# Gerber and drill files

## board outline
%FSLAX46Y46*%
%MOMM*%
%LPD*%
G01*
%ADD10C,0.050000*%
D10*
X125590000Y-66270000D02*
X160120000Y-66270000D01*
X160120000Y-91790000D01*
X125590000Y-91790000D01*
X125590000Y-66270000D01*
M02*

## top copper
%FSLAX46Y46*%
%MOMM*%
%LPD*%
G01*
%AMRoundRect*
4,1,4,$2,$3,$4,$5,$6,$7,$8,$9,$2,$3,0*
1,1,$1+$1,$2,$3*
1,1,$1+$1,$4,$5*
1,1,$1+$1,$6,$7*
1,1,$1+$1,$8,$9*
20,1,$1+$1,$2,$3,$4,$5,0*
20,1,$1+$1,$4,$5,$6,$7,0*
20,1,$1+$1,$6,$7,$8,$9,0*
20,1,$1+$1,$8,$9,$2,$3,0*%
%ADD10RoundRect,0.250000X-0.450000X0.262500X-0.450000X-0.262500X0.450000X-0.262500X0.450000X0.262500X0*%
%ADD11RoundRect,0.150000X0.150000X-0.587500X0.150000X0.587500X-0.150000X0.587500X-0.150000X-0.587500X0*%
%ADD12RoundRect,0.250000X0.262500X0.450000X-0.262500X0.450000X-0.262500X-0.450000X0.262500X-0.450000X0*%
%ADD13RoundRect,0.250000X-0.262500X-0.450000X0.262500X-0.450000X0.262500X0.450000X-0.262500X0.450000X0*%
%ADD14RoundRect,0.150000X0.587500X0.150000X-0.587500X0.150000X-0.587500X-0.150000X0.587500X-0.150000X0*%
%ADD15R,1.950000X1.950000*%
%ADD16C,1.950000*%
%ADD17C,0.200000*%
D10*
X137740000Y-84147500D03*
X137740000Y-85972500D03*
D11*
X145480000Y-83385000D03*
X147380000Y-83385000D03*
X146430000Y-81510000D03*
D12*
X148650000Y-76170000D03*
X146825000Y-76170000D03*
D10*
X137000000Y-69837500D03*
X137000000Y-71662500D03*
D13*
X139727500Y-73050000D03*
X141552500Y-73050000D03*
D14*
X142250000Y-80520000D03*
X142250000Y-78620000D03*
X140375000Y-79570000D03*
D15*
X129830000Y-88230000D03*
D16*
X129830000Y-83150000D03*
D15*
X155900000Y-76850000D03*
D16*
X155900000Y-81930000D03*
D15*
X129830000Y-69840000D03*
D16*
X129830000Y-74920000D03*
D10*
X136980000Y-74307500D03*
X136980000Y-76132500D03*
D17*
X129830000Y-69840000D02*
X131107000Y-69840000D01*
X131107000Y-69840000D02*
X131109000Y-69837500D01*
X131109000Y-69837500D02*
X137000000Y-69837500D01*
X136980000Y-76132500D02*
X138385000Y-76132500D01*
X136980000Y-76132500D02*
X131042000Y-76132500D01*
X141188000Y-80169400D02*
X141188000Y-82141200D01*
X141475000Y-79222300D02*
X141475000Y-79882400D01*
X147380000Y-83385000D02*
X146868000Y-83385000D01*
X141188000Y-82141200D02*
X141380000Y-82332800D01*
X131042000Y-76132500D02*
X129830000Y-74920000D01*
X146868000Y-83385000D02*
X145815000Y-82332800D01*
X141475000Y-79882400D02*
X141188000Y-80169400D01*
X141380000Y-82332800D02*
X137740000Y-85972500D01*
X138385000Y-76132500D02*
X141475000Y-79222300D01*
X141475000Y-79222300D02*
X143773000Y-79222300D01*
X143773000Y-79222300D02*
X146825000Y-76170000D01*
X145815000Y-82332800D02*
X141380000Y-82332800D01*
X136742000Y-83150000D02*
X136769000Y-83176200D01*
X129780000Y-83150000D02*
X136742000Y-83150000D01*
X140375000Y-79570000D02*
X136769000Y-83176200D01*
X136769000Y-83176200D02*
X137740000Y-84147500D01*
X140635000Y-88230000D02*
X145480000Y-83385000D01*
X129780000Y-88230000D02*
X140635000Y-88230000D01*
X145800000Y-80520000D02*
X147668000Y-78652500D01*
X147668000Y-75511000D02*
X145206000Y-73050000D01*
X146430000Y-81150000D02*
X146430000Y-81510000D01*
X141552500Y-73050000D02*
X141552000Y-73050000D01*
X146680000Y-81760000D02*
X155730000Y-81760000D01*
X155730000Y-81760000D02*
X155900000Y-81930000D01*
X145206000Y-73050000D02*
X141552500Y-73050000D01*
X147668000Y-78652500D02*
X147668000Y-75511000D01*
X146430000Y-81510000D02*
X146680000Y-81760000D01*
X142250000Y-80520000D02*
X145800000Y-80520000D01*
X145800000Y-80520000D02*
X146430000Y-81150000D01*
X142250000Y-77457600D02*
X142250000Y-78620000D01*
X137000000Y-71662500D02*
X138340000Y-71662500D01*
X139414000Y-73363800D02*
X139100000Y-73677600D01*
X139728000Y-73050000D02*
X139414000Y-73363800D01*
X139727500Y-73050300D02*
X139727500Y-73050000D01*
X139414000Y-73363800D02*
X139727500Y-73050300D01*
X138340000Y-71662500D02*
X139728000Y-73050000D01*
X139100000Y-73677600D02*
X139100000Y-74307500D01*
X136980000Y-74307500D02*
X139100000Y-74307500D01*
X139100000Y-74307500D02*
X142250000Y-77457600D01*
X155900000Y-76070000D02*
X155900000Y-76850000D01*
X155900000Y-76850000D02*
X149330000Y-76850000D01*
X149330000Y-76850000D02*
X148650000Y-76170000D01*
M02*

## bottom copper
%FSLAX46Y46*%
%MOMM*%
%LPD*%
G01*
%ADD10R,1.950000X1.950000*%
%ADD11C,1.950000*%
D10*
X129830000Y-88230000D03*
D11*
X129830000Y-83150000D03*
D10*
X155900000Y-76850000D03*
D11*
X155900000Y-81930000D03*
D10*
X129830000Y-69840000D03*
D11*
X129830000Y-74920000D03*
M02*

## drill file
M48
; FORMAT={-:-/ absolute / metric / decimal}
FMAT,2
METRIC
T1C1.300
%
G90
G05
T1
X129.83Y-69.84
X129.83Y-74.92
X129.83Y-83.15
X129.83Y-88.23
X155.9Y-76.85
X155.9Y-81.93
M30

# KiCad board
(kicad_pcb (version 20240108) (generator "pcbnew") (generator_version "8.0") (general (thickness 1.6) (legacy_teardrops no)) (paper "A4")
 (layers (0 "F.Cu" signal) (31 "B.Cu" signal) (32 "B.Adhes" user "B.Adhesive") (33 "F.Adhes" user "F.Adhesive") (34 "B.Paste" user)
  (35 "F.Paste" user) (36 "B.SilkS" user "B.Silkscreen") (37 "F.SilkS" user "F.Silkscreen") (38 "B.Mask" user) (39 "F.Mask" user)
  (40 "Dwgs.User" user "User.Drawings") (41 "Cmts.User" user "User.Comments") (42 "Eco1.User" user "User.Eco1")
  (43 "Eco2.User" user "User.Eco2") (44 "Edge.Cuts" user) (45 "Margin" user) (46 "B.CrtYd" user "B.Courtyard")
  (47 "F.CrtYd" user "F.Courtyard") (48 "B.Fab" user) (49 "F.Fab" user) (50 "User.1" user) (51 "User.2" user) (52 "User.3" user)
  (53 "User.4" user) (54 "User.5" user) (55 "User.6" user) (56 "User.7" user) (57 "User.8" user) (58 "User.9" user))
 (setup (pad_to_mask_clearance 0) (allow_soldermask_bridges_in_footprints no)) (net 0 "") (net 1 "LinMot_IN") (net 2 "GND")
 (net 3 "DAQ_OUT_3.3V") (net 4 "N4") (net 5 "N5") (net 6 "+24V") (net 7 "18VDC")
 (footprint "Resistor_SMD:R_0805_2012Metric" (layer "F.Cu") (at 137.74 85.06 -90)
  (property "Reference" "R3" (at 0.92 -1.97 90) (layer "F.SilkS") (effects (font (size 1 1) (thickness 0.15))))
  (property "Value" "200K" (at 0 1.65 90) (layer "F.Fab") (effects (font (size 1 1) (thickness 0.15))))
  (pad "1" smd roundrect (at -0.9125 0 270) (size 1.025 1.4) (layers "F.Cu" "F.Paste" "F.Mask") (roundrect_rratio 0.243902)
   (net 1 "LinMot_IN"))
  (pad "2" smd roundrect (at 0.9125 0 270) (size 1.025 1.4) (layers "F.Cu" "F.Paste" "F.Mask") (roundrect_rratio 0.243902) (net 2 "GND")))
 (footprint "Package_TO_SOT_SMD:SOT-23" (layer "F.Cu") (at 146.43 82.4475 90)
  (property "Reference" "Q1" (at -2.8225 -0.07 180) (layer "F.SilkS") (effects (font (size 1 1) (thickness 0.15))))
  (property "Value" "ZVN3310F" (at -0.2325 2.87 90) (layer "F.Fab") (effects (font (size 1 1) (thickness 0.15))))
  (pad "1" smd roundrect (at -0.9375 -0.95 90) (size 1.475 0.6) (layers "F.Cu" "F.Paste" "F.Mask") (roundrect_rratio 0.25)
   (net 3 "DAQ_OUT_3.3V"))
  (pad "2" smd roundrect (at -0.9375 0.95 90) (size 1.475 0.6) (layers "F.Cu" "F.Paste" "F.Mask") (roundrect_rratio 0.25) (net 2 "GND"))
  (pad "3" smd roundrect (at 0.9375 0 90) (size 1.475 0.6) (layers "F.Cu" "F.Paste" "F.Mask") (roundrect_rratio 0.25) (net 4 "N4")))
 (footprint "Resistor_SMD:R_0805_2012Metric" (layer "F.Cu") (at 147.7375 76.17 180)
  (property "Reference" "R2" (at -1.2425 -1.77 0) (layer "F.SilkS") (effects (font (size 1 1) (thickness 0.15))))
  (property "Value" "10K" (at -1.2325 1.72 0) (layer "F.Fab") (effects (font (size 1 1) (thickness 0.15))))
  (pad "1" smd roundrect (at -0.9125 0 180) (size 1.025 1.4) (layers "F.Cu" "F.Paste" "F.Mask") (roundrect_rratio 0.243902) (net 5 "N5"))
  (pad "2" smd roundrect (at 0.9125 0 180) (size 1.025 1.4) (layers "F.Cu" "F.Paste" "F.Mask") (roundrect_rratio 0.243902) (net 2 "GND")))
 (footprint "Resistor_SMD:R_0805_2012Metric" (layer "F.Cu") (at 137 70.75 -90)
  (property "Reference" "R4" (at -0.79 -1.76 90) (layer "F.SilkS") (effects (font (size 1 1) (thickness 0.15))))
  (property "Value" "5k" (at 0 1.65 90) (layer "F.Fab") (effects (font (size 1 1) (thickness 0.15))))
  (pad "1" smd roundrect (at -0.9125 0 270) (size 1.025 1.4) (layers "F.Cu" "F.Paste" "F.Mask") (roundrect_rratio 0.243902) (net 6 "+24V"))
  (pad "2" smd roundrect (at 0.9125 0 270) (size 1.025 1.4) (layers "F.Cu" "F.Paste" "F.Mask") (roundrect_rratio 0.243902) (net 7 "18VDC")))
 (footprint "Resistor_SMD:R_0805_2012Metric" (layer "F.Cu") (at 140.64 73.05)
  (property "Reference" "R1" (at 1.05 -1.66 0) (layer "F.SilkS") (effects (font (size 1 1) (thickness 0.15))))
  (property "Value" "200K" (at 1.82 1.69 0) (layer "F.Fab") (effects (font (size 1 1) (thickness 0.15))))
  (pad "1" smd roundrect (at -0.9125 0) (size 1.025 1.4) (layers "F.Cu" "F.Paste" "F.Mask") (roundrect_rratio 0.243902) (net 7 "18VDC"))
  (pad "2" smd roundrect (at 0.9125 0) (size 1.025 1.4) (layers "F.Cu" "F.Paste" "F.Mask") (roundrect_rratio 0.243902) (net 4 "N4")))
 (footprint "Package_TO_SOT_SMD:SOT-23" (layer "F.Cu") (at 141.3125 79.57 180)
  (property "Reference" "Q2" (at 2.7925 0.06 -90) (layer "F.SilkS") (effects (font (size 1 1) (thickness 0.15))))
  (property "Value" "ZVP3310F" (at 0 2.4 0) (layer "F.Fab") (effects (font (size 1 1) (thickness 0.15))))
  (pad "1" smd roundrect (at -0.9375 -0.95 180) (size 1.475 0.6) (layers "F.Cu" "F.Paste" "F.Mask") (roundrect_rratio 0.25) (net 4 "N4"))
  (pad "2" smd roundrect (at -0.9375 0.95 180) (size 1.475 0.6) (layers "F.Cu" "F.Paste" "F.Mask") (roundrect_rratio 0.25) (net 7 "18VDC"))
  (pad "3" smd roundrect (at 0.9375 0 180) (size 1.475 0.6) (layers "F.Cu" "F.Paste" "F.Mask") (roundrect_rratio 0.25) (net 1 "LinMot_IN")))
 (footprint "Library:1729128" (layer "F.Cu") (at 129.83 88.23 90)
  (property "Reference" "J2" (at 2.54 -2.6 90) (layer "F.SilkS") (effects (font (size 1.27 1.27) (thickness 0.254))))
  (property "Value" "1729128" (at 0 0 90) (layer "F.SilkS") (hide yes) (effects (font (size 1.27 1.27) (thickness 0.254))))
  (pad "1" thru_hole rect (at 0 0 90) (size 1.95 1.95) (drill 1.3) (layers "*.Cu" "*.Mask") (remove_unused_layers no) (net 3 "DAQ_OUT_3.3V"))
  (pad "2" thru_hole circle (at 5.08 0 90) (size 1.95 1.95) (drill 1.3) (layers "*.Cu" "*.Mask") (remove_unused_layers no)
   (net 1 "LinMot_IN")))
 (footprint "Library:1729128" (layer "F.Cu") (at 155.9 76.85 -90)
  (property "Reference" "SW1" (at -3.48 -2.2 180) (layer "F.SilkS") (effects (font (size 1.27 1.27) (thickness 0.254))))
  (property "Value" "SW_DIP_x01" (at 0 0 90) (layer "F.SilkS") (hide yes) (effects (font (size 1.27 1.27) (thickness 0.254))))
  (pad "1" thru_hole rect (at 0 0 270) (size 1.95 1.95) (drill 1.3) (layers "*.Cu" "*.Mask") (remove_unused_layers no) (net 5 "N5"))
  (pad "2" thru_hole circle (at 5.08 0 270) (size 1.95 1.95) (drill 1.3) (layers "*.Cu" "*.Mask") (remove_unused_layers no) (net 4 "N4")))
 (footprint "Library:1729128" (layer "F.Cu") (at 129.83 69.84 -90)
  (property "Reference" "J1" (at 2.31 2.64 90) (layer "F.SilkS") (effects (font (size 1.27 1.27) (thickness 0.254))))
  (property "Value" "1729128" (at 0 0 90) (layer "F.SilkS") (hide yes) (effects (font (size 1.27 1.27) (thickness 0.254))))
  (pad "1" thru_hole rect (at 0 0 270) (size 1.95 1.95) (drill 1.3) (layers "*.Cu" "*.Mask") (remove_unused_layers no) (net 6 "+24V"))
  (pad "2" thru_hole circle (at 5.08 0 270) (size 1.95 1.95) (drill 1.3) (layers "*.Cu" "*.Mask") (remove_unused_layers no) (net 2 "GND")))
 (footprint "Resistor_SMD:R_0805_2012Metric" (layer "F.Cu") (at 136.98 75.22 -90)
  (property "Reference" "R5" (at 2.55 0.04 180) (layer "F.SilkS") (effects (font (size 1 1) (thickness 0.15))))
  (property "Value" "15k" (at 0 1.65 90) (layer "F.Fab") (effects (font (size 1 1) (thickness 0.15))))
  (pad "1" smd roundrect (at -0.9125 0 270) (size 1.025 1.4) (layers "F.Cu" "F.Paste" "F.Mask") (roundrect_rratio 0.243902) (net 7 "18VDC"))
  (pad "2" smd roundrect (at 0.9125 0 270) (size 1.025 1.4) (layers "F.Cu" "F.Paste" "F.Mask") (roundrect_rratio 0.243902) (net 2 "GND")))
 (gr_rect (start 125.59 66.27) (end 160.12 91.79) (stroke (width 0.05) (type default)) (fill none) (layer "Edge.Cuts"))
 (segment (start 129.83 69.84) (end 131.107 69.84) (width 0.2) (layer "F.Cu") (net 6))
 (segment (start 131.107 69.84) (end 131.109 69.8375) (width 0.2) (layer "F.Cu") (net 6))
 (segment (start 131.109 69.8375) (end 137 69.8375) (width 0.2) (layer "F.Cu") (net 6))
 (segment (start 136.98 76.1325) (end 138.385 76.1325) (width 0.2) (layer "F.Cu") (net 2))
 (segment (start 136.98 76.1325) (end 131.042 76.1325) (width 0.2) (layer "F.Cu") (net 2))
 (segment (start 141.188 80.1694) (end 141.188 82.1412) (width 0.2) (layer "F.Cu") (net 2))
 (segment (start 141.475 79.2223) (end 141.475 79.8824) (width 0.2) (layer "F.Cu") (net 2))
 (segment (start 147.38 83.385) (end 146.868 83.385) (width 0.2) (layer "F.Cu") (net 2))
 (segment (start 141.188 82.1412) (end 141.38 82.3328) (width 0.2) (layer "F.Cu") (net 2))
 (segment (start 131.042 76.1325) (end 129.83 74.92) (width 0.2) (layer "F.Cu") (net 2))
 (segment (start 146.868 83.385) (end 145.815 82.3328) (width 0.2) (layer "F.Cu") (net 2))
 (segment (start 141.475 79.8824) (end 141.188 80.1694) (width 0.2) (layer "F.Cu") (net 2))
 (segment (start 141.38 82.3328) (end 137.74 85.9725) (width 0.2) (layer "F.Cu") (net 2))
 (segment (start 138.385 76.1325) (end 141.475 79.2223) (width 0.2) (layer "F.Cu") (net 2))
 (segment (start 141.475 79.2223) (end 143.773 79.2223) (width 0.2) (layer "F.Cu") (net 2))
 (segment (start 143.773 79.2223) (end 146.825 76.17) (width 0.2) (layer "F.Cu") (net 2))
 (segment (start 145.815 82.3328) (end 141.38 82.3328) (width 0.2) (layer "F.Cu") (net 2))
 (segment (start 136.742 83.15) (end 136.769 83.1762) (width 0.2) (layer "F.Cu") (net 1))
 (segment (start 129.78 83.15) (end 136.742 83.15) (width 0.2) (layer "F.Cu") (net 1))
 (segment (start 140.375 79.57) (end 136.769 83.1762) (width 0.2) (layer "F.Cu") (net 1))
 (segment (start 136.769 83.1762) (end 137.74 84.1475) (width 0.2) (layer "F.Cu") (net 1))
 (segment (start 140.635 88.23) (end 145.48 83.385) (width 0.2) (layer "F.Cu") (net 3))
 (segment (start 129.78 88.23) (end 140.635 88.23) (width 0.2) (layer "F.Cu") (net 3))
 (segment (start 145.8 80.52) (end 147.668 78.6525) (width 0.2) (layer "F.Cu") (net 4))
 (segment (start 147.668 75.511) (end 145.206 73.05) (width 0.2) (layer "F.Cu") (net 4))
 (segment (start 146.43 81.15) (end 146.43 81.51) (width 0.2) (layer "F.Cu") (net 4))
 (segment (start 141.5525 73.05) (end 141.552 73.05) (width 0.2) (layer "F.Cu") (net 4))
 (segment (start 146.68 81.76) (end 155.73 81.76) (width 0.2) (layer "F.Cu") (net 4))
 (segment (start 155.73 81.76) (end 155.9 81.93) (width 0.2) (layer "F.Cu") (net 4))
 (segment (start 145.206 73.05) (end 141.5525 73.05) (width 0.2) (layer "F.Cu") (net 4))
 (segment (start 147.668 78.6525) (end 147.668 75.511) (width 0.2) (layer "F.Cu") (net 4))
 (segment (start 146.43 81.51) (end 146.68 81.76) (width 0.2) (layer "F.Cu") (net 4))
 (segment (start 142.25 80.52) (end 145.8 80.52) (width 0.2) (layer "F.Cu") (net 4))
 (segment (start 145.8 80.52) (end 146.43 81.15) (width 0.2) (layer "F.Cu") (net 4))
 (segment (start 142.25 77.4576) (end 142.25 78.62) (width 0.2) (layer "F.Cu") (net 7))
 (segment (start 137 71.6625) (end 138.34 71.6625) (width 0.2) (layer "F.Cu") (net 7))
 (segment (start 139.414 73.3638) (end 139.1 73.6776) (width 0.2) (layer "F.Cu") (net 7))
 (segment (start 139.728 73.05) (end 139.414 73.3638) (width 0.2) (layer "F.Cu") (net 7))
 (segment (start 139.7275 73.0503) (end 139.7275 73.05) (width 0.2) (layer "F.Cu") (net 7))
 (segment (start 139.414 73.3638) (end 139.7275 73.0503) (width 0.2) (layer "F.Cu") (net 7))
 (segment (start 138.34 71.6625) (end 139.728 73.05) (width 0.2) (layer "F.Cu") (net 7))
 (segment (start 139.1 73.6776) (end 139.1 74.3075) (width 0.2) (layer "F.Cu") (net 7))
 (segment (start 136.98 74.3075) (end 139.1 74.3075) (width 0.2) (layer "F.Cu") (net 7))
 (segment (start 139.1 74.3075) (end 142.25 77.4576) (width 0.2) (layer "F.Cu") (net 7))
 (segment (start 155.9 76.07) (end 155.9 76.85) (width 0.2) (layer "F.Cu") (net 5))
 (segment (start 155.9 76.85) (end 149.33 76.85) (width 0.2) (layer "F.Cu") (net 5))
 (segment (start 149.33 76.85) (end 148.65 76.17) (width 0.2) (layer "F.Cu") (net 5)))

